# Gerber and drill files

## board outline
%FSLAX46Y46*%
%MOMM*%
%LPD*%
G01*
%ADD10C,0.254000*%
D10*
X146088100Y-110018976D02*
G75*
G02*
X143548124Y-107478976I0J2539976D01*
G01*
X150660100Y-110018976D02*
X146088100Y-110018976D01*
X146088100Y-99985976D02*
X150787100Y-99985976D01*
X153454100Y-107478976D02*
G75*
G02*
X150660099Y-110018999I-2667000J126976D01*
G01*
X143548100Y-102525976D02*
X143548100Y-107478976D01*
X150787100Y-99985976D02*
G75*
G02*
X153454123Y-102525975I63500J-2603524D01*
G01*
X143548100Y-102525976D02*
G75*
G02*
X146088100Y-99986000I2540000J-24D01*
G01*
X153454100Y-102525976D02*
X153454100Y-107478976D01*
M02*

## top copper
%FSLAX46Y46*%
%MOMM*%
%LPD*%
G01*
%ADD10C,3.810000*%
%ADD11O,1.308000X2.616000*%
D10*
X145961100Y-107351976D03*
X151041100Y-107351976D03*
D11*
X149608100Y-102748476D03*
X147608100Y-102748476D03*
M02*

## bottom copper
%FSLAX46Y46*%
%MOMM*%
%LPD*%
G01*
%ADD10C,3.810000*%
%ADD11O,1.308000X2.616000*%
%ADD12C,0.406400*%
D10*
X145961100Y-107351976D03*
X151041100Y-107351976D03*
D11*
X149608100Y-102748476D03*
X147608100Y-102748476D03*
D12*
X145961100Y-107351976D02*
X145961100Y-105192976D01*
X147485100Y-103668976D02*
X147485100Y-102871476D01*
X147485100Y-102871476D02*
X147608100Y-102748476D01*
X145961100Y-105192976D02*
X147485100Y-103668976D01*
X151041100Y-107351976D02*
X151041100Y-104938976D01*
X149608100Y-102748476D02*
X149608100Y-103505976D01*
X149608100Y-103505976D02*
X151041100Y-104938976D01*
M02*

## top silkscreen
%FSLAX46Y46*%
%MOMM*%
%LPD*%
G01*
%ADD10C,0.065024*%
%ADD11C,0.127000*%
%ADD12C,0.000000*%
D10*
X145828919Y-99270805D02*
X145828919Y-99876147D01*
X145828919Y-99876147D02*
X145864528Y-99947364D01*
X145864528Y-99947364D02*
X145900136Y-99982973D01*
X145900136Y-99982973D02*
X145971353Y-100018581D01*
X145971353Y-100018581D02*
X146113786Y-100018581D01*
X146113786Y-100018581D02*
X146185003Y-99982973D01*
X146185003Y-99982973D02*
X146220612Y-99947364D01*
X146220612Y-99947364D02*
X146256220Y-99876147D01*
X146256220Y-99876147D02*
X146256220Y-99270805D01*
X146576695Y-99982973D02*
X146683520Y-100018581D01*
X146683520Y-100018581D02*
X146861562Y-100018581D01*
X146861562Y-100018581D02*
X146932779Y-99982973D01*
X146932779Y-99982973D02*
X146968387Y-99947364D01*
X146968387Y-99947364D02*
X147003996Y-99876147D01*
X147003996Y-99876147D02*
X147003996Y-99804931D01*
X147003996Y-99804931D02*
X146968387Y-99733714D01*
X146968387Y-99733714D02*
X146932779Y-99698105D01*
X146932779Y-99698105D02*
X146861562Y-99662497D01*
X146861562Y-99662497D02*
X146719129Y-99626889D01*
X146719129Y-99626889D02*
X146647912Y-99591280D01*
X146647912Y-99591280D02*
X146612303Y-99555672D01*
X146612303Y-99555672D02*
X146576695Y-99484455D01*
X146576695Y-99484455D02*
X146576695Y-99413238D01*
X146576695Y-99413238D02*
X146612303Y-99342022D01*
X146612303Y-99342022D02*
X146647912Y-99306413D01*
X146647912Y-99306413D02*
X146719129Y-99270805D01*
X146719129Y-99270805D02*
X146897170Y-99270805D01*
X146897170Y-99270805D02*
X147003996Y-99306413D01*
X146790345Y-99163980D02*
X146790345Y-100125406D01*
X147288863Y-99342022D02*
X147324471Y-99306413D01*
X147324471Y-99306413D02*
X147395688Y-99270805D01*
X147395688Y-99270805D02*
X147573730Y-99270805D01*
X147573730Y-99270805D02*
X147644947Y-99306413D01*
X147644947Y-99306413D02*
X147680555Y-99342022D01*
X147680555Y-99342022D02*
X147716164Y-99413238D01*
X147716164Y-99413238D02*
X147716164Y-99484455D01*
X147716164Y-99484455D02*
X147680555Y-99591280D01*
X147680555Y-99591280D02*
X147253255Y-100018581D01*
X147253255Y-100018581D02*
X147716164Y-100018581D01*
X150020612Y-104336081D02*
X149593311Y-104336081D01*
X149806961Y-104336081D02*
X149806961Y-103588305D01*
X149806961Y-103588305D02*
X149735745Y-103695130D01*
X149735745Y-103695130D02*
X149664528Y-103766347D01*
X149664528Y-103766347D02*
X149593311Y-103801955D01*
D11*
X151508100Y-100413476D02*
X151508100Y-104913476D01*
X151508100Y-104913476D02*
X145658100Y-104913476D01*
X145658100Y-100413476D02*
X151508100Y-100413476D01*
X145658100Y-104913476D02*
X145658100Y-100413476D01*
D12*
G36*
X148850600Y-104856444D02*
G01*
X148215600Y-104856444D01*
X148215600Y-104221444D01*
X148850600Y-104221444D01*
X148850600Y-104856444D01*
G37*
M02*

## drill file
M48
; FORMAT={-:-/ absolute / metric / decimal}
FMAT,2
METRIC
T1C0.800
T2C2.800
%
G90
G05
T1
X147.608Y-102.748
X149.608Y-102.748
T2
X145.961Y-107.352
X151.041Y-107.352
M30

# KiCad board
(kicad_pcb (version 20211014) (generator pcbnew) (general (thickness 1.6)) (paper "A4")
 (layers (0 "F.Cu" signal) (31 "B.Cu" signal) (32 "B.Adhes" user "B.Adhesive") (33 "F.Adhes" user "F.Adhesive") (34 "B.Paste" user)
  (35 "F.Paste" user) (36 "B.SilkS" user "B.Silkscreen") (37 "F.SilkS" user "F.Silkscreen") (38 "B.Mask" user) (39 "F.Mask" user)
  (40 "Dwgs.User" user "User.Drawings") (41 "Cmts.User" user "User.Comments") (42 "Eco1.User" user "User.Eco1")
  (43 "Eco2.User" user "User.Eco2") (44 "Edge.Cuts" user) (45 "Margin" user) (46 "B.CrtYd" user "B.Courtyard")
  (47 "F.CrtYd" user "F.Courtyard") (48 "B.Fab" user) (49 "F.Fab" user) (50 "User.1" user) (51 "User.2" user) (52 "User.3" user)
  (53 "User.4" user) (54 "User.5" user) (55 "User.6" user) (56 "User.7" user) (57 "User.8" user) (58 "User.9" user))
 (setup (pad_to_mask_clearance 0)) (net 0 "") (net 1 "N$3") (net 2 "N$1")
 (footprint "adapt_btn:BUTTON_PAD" (layer "F.Cu") (at 145.9611 107.351976)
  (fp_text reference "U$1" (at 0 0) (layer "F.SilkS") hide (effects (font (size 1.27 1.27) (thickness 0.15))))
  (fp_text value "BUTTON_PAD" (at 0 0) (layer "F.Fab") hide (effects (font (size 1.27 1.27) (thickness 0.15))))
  (pad "P$1" thru_hole circle (at 0 0) (size 3.81 3.81) (drill 2.8) (layers *.Cu *.Mask) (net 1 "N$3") (solder_mask_margin 0.1016)))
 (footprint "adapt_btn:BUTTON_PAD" (layer "F.Cu") (at 151.0411 107.351976)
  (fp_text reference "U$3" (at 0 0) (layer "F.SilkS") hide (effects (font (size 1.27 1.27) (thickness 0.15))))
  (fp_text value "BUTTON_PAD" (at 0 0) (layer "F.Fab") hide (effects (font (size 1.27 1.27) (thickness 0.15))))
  (pad "P$1" thru_hole circle (at 0 0) (size 3.81 3.81) (drill 2.8) (layers *.Cu *.Mask) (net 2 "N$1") (solder_mask_margin 0.1016)))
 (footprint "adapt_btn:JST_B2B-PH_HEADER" (layer "F.Cu") (at 148.5331 102.795976)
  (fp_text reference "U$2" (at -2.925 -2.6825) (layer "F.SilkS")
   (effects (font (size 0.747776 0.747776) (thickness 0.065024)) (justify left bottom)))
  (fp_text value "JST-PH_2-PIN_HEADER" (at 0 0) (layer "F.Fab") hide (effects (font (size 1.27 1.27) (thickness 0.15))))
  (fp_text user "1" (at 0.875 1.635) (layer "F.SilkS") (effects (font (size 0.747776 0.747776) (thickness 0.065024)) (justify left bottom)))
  (fp_line (start 2.975 -2.3825) (end 2.975 2.1175) (layer "F.SilkS") (width 0.127))
  (fp_line (start 2.975 2.1175) (end -2.875 2.1175) (layer "F.SilkS") (width 0.127))
  (fp_line (start -2.875 -2.3825) (end 2.975 -2.3825) (layer "F.SilkS") (width 0.127))
  (fp_line (start -2.875 2.1175) (end -2.875 -2.3825) (layer "F.SilkS") (width 0.127))
  (fp_poly
   (pts (xy -0.3175 2.060468) (xy 0.3175 2.060468) (xy 0.3175 1.425468) (xy -0.3175 1.425468)) (layer "F.SilkS") (width 0) (fill solid))
  (pad "P1" thru_hole oval (at 1.075 -0.0475 90) (size 2.616 1.308) (drill 0.8) (layers *.Cu *.Mask) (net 2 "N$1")
   (solder_mask_margin 0.1016))
  (pad "P2" thru_hole oval (at -0.925 -0.0475 90) (size 2.616 1.308) (drill 0.8) (layers *.Cu *.Mask) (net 1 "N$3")
   (solder_mask_margin 0.1016)))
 (gr_arc (start 146.0881 110.018976) (mid 144.292049 109.275027) (end 143.5481 107.478976) (layer "Edge.Cuts") (width 0.254))
 (gr_line (start 150.6601 110.018976) (end 146.0881 110.018976) (layer "Edge.Cuts") (width 0.254))
 (gr_line (start 146.0881 99.985976) (end 150.7871 99.985976) (layer "Edge.Cuts") (width 0.254))
 (gr_arc (start 153.4541 107.478976) (mid 152.583151 109.327632) (end 150.6601 110.018976) (layer "Edge.Cuts") (width 0.254))
 (gr_line (start 143.5481 102.525976) (end 143.5481 107.478976) (layer "Edge.Cuts") (width 0.254))
 (gr_arc (start 150.7871 99.985976) (mid 152.646651 100.703622) (end 153.4541 102.525976) (layer "Edge.Cuts") (width 0.254))
 (gr_arc (start 143.5481 102.525976) (mid 144.292049 100.729925) (end 146.0881 99.985976) (layer "Edge.Cuts") (width 0.254))
 (gr_line (start 153.4541 102.525976) (end 153.4541 107.478976) (layer "Edge.Cuts") (width 0.254))
 (segment (start 145.9611 107.351976) (end 145.9611 105.192976) (width 0.4064) (layer "B.Cu") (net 1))
 (segment (start 147.4851 103.668976) (end 147.4851 102.871476) (width 0.4064) (layer "B.Cu") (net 1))
 (segment (start 147.4851 102.871476) (end 147.6081 102.748476) (width 0.4064) (layer "B.Cu") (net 1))
 (segment (start 145.9611 105.192976) (end 147.4851 103.668976) (width 0.4064) (layer "B.Cu") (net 1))
 (segment (start 151.0411 107.351976) (end 151.0411 104.938976) (width 0.4064) (layer "B.Cu") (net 2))
 (segment (start 149.6081 102.748476) (end 149.6081 103.505976) (width 0.4064) (layer "B.Cu") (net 2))
 (segment (start 149.6081 103.505976) (end 151.0411 104.938976) (width 0.4064) (layer "B.Cu") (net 2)))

